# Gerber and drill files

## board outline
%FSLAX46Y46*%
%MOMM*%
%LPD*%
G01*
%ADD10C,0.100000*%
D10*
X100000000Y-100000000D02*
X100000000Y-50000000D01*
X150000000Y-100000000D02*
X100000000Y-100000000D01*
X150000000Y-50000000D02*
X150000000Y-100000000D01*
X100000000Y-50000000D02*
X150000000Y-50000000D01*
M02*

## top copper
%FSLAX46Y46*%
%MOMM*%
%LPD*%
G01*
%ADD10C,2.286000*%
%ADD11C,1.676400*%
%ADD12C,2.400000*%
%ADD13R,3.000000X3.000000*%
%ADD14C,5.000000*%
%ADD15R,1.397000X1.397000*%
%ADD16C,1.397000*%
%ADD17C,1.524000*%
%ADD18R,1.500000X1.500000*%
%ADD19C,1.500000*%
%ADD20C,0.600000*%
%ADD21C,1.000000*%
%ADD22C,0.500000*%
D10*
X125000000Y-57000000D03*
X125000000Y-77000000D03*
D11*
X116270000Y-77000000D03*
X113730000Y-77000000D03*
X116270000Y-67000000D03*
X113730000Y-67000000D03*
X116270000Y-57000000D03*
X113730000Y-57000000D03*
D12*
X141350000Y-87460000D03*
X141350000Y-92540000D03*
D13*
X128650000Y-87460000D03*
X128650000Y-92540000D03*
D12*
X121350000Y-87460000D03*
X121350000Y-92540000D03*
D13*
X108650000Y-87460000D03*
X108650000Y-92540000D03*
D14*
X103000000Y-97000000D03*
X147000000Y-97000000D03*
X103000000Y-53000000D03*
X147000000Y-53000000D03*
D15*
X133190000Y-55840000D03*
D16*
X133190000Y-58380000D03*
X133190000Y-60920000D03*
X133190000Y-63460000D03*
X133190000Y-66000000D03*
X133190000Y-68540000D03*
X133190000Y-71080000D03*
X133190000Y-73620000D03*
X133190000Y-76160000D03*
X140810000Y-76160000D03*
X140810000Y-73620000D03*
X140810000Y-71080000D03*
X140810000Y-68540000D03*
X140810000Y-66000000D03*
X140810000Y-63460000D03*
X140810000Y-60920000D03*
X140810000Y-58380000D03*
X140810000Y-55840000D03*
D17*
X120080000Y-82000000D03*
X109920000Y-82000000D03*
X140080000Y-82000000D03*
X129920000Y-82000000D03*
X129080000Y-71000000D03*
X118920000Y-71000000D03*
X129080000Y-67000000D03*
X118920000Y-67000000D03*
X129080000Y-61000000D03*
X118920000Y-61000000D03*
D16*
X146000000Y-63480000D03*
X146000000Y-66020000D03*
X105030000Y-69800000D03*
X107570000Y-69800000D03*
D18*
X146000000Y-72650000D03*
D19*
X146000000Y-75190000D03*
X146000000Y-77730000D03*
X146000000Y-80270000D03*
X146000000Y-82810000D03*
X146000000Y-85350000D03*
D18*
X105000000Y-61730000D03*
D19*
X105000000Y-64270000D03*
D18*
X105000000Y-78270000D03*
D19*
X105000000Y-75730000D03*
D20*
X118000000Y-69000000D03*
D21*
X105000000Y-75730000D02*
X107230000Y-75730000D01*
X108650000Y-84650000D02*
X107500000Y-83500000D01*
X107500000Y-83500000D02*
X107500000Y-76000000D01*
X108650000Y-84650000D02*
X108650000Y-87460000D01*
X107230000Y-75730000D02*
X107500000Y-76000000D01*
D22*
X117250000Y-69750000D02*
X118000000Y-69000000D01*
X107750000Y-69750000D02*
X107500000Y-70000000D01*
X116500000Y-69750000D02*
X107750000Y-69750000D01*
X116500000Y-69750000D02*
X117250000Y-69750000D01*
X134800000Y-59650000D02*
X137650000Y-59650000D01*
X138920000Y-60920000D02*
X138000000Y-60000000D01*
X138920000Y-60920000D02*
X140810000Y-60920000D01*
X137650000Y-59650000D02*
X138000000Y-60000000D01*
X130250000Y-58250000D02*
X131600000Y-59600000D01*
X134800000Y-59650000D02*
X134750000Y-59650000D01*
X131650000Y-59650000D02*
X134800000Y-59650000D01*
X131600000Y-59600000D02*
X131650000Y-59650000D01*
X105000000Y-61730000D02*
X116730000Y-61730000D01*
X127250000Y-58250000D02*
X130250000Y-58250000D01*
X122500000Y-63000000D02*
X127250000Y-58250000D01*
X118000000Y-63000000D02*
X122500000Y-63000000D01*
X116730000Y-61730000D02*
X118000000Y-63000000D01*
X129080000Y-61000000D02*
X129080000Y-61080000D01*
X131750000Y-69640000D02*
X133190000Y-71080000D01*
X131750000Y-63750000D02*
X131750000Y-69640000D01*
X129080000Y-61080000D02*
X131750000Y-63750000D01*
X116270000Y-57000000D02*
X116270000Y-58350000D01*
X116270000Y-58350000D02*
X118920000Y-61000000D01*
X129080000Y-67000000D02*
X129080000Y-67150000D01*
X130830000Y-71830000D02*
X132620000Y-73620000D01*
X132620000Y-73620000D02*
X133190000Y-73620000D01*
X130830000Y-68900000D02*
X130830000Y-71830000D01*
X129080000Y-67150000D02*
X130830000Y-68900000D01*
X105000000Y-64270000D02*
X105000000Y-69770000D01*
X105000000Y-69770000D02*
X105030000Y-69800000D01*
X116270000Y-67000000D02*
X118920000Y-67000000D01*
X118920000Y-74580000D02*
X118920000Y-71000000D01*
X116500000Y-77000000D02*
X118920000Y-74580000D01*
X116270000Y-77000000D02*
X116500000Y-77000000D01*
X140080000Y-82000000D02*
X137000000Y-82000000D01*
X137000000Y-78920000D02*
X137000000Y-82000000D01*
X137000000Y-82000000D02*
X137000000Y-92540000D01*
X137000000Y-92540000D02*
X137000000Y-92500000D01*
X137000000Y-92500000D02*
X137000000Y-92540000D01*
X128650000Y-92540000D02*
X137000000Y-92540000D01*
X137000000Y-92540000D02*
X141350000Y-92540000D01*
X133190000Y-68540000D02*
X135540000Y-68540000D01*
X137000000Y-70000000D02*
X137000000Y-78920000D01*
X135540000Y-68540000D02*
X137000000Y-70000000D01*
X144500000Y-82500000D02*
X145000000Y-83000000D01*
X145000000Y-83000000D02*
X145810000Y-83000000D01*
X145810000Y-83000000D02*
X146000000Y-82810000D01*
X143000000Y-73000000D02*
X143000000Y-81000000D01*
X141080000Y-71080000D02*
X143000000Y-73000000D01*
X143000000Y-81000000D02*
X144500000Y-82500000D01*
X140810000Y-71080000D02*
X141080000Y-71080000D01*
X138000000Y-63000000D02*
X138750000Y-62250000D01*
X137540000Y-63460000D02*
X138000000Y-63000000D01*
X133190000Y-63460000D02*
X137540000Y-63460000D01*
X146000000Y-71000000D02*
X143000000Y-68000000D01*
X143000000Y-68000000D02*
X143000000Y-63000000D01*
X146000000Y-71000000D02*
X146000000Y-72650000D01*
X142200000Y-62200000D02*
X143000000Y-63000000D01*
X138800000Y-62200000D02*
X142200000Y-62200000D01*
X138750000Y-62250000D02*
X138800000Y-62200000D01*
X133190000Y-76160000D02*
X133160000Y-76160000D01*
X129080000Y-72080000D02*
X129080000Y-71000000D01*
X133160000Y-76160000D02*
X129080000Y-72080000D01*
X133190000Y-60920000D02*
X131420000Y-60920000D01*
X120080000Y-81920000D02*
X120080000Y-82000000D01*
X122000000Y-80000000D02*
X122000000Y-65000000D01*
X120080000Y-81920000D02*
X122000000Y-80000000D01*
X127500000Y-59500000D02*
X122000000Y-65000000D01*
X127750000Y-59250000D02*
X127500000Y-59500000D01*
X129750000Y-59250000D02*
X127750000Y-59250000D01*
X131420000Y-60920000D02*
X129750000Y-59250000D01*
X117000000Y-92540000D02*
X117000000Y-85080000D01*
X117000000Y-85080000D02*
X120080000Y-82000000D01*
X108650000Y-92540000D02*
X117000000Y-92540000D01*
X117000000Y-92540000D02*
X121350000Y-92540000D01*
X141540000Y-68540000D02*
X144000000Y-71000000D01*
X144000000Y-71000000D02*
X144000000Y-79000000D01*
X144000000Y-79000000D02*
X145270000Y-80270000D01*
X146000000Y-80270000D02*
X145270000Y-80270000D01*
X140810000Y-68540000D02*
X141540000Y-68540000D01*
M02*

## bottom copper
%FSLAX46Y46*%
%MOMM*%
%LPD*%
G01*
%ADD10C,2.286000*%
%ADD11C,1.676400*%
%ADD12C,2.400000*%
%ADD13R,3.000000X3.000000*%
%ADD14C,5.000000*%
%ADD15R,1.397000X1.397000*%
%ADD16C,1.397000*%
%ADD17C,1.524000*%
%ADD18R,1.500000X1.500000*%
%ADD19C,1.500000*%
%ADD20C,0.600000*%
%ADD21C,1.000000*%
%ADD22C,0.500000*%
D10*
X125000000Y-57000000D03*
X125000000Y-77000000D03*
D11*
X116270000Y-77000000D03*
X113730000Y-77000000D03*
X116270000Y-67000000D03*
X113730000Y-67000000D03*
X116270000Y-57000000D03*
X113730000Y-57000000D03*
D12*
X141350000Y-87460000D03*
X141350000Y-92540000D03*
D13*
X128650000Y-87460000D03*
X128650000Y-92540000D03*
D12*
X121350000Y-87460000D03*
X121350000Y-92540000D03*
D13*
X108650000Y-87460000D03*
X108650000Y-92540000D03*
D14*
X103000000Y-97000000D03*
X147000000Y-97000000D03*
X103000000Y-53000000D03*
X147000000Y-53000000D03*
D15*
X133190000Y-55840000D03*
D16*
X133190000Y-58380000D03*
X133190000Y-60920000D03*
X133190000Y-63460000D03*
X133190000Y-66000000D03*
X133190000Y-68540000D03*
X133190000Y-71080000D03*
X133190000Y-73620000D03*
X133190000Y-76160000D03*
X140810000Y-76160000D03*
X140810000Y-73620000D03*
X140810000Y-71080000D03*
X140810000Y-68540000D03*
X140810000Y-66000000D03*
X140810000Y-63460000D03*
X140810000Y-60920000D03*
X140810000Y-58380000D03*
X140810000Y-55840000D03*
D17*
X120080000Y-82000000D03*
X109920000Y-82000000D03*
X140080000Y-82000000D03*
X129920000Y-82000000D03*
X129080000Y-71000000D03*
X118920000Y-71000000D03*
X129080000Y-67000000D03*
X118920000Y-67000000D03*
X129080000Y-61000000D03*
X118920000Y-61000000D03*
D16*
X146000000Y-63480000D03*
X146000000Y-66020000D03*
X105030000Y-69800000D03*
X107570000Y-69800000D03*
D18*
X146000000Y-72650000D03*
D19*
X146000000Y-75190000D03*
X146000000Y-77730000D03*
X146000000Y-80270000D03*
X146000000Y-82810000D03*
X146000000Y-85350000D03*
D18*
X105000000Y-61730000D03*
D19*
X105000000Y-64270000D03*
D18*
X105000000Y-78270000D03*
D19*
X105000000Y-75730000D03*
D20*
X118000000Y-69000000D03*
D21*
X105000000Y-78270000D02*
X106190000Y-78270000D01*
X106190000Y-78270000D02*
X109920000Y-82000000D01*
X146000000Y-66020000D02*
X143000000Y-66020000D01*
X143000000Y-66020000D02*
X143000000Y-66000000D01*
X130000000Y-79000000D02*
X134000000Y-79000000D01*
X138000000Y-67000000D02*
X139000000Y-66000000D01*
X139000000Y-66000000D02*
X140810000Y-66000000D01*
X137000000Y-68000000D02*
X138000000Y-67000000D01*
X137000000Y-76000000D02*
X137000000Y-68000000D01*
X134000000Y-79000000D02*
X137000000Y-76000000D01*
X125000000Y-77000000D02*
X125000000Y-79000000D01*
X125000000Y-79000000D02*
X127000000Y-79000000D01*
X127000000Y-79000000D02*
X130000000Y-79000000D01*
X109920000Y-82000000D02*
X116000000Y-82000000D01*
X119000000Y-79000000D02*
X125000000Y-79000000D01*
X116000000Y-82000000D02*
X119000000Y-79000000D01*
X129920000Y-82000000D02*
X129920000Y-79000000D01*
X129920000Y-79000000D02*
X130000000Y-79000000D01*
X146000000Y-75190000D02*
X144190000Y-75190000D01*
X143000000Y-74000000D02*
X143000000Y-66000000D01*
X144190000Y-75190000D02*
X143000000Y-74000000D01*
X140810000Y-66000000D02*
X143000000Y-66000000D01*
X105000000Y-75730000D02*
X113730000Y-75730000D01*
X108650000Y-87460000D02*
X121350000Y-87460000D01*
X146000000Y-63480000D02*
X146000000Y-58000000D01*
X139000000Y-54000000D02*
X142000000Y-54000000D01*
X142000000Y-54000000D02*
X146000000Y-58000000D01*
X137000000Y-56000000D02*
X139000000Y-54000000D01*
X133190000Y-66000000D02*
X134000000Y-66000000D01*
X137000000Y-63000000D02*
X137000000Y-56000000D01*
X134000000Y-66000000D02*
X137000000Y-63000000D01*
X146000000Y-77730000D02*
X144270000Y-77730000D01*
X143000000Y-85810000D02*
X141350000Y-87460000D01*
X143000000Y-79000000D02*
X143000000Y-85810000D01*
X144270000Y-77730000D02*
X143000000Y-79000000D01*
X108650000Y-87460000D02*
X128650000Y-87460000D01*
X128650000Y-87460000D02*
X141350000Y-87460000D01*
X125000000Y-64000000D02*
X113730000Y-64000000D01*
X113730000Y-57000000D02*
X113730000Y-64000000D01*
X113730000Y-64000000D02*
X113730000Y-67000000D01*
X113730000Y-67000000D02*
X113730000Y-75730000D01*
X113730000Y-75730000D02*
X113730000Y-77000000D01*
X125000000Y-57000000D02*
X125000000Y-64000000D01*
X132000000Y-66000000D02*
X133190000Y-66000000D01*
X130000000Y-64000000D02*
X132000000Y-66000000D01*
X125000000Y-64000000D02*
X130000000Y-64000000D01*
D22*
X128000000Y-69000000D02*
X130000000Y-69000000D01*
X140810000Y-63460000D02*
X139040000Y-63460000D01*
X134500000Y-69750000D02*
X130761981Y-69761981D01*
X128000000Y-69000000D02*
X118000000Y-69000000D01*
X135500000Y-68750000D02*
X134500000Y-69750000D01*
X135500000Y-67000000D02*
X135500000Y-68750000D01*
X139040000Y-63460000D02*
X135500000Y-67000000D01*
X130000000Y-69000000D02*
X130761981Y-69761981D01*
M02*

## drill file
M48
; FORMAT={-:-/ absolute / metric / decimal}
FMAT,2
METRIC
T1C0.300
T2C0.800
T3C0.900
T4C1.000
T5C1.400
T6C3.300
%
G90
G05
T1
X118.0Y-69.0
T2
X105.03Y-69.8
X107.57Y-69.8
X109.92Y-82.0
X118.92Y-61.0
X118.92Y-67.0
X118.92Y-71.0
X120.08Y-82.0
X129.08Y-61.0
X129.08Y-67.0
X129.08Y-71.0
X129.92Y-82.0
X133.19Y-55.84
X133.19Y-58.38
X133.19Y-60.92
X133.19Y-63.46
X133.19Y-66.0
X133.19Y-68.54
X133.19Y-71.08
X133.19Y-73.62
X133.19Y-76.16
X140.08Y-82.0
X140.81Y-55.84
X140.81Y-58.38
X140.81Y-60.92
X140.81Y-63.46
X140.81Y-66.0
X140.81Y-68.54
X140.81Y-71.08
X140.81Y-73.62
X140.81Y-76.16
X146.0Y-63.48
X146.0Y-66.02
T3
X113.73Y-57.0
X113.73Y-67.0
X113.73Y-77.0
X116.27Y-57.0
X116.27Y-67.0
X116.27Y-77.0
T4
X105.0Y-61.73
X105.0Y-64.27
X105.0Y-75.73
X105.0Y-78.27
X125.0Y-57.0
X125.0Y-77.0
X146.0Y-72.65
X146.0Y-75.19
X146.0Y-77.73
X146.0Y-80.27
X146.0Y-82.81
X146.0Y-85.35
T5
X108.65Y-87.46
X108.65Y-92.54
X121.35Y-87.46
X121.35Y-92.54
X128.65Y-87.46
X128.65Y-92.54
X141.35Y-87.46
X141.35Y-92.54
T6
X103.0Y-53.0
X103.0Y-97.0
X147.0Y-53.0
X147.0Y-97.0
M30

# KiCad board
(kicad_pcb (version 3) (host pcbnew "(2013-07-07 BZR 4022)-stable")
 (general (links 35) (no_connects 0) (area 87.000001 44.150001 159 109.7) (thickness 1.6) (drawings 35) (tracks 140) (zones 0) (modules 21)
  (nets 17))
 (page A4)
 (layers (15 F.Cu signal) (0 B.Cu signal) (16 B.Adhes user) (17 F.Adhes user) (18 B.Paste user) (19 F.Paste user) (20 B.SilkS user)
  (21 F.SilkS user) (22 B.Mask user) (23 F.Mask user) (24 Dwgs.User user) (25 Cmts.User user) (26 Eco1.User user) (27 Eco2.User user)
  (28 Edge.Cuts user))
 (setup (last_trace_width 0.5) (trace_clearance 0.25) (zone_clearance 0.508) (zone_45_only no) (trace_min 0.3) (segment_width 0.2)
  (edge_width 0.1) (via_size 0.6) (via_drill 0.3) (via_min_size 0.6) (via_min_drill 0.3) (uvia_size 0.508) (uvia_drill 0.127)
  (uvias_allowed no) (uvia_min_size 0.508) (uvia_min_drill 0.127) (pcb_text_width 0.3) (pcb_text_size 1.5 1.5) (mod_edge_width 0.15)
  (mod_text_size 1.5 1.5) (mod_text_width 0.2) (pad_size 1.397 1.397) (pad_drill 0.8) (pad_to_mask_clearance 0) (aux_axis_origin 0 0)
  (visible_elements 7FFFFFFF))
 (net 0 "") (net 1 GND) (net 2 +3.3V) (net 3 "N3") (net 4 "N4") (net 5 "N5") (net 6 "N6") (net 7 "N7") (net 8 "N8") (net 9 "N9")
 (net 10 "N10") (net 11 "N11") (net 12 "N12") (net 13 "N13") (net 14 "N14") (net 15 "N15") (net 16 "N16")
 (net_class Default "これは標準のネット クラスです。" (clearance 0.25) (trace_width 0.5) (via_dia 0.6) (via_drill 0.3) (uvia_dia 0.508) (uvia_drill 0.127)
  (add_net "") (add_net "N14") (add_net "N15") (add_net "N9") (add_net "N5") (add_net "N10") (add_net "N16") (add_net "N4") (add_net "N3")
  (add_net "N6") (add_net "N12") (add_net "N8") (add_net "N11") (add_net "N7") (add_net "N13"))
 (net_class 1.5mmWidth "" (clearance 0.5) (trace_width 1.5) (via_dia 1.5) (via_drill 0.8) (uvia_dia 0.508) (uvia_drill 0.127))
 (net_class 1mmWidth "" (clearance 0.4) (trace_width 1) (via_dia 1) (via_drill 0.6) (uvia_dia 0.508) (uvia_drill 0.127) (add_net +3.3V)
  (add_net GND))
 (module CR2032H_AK (layer B.Cu) (at 125 62 270)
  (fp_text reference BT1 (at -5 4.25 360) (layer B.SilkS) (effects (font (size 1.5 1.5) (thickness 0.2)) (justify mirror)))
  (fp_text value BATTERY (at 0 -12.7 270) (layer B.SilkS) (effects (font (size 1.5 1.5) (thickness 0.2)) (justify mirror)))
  (pad 2 thru_hole circle (at -5 0 270) (size 2.286 2.286) (drill 1) (layers *.Cu *.Mask B.SilkS) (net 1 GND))
  (pad 1 thru_hole circle (at 15 0 270) (size 2.286 2.286) (drill 1) (layers *.Cu *.Mask B.SilkS) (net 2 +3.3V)))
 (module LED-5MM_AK (layer F.Cu) (at 115 77 180)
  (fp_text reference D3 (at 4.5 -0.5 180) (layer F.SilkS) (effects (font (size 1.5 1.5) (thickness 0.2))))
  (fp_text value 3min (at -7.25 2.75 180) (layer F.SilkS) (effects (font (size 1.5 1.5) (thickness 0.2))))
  (pad 1 thru_hole circle (at -1.27 0 180) (size 1.6764 1.6764) (drill 0.9) (layers *.Cu *.Mask F.SilkS) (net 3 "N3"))
  (pad 2 thru_hole circle (at 1.27 0 180) (size 1.6764 1.6764) (drill 0.9) (layers *.Cu *.Mask F.SilkS) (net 1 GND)))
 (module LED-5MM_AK (layer F.Cu) (at 115 67 180)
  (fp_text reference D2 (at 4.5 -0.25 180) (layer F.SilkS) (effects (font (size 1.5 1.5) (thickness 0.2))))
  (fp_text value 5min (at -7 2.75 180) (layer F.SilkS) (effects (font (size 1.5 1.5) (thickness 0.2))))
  (pad 1 thru_hole circle (at -1.27 0 180) (size 1.6764 1.6764) (drill 0.9) (layers *.Cu *.Mask F.SilkS) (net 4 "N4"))
  (pad 2 thru_hole circle (at 1.27 0 180) (size 1.6764 1.6764) (drill 0.9) (layers *.Cu *.Mask F.SilkS) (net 1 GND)))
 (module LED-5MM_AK (layer F.Cu) (at 115 57 180)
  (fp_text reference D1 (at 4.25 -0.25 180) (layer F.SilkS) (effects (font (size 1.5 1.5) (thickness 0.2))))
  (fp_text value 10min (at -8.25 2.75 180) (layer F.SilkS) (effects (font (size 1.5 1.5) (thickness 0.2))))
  (pad 1 thru_hole circle (at -1.27 0 180) (size 1.6764 1.6764) (drill 0.9) (layers *.Cu *.Mask F.SilkS) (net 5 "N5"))
  (pad 2 thru_hole circle (at 1.27 0 180) (size 1.6764 1.6764) (drill 0.9) (layers *.Cu *.Mask F.SilkS) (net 1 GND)))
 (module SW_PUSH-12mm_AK (layer F.Cu) (at 135 90)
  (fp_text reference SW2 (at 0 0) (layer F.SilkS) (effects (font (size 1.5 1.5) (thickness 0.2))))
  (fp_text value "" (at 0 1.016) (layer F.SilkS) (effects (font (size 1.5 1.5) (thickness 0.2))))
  (pad 1 thru_hole circle (at 6.35 -2.54) (size 2.4 2.4) (drill 1.4) (layers *.Cu *.Mask F.SilkS) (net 1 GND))
  (pad 2 thru_hole circle (at 6.35 2.54) (size 2.4 2.4) (drill 1.4) (layers *.Cu *.Mask F.SilkS) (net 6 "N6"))
  (pad 1 thru_hole rect (at -6.35 -2.54) (size 3 3) (drill 1.4) (layers *.Cu *.Mask F.SilkS) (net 1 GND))
  (pad 2 thru_hole rect (at -6.35 2.54) (size 3 3) (drill 1.4) (layers *.Cu *.Mask F.SilkS) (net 6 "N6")))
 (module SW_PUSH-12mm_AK (layer F.Cu) (at 115 90)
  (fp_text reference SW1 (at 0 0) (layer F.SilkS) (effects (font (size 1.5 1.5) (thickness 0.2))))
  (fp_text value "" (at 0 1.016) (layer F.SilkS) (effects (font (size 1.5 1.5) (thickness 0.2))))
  (pad 1 thru_hole circle (at 6.35 -2.54) (size 2.4 2.4) (drill 1.4) (layers *.Cu *.Mask F.SilkS) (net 1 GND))
  (pad 2 thru_hole circle (at 6.35 2.54) (size 2.4 2.4) (drill 1.4) (layers *.Cu *.Mask F.SilkS) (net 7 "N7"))
  (pad 1 thru_hole rect (at -6.35 -2.54) (size 3 3) (drill 1.4) (layers *.Cu *.Mask F.SilkS) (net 1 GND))
  (pad 2 thru_hole rect (at -6.35 2.54) (size 3 3) (drill 1.4) (layers *.Cu *.Mask F.SilkS) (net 7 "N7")))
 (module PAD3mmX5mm (layer F.Cu) (at 103 97)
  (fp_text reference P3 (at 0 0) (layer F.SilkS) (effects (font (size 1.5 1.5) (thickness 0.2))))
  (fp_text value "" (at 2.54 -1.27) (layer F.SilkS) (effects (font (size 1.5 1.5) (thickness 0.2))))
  (pad "" thru_hole circle (at 0 0) (size 5 5) (drill 3.3) (layers *.Cu *.Mask F.SilkS)))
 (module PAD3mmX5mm (layer F.Cu) (at 147 97)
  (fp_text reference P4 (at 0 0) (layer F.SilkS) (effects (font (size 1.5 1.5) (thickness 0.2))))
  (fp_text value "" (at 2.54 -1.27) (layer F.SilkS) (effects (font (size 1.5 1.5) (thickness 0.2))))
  (pad "" thru_hole circle (at 0 0) (size 5 5) (drill 3.3) (layers *.Cu *.Mask F.SilkS)))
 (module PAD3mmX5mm (layer F.Cu) (at 103 53)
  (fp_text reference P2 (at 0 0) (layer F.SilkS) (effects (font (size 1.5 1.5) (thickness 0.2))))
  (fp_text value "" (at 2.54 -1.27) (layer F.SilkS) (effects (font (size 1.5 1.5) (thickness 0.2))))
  (pad "" thru_hole circle (at 0 0) (size 5 5) (drill 3.3) (layers *.Cu *.Mask F.SilkS)))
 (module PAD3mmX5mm (layer F.Cu) (at 147 53)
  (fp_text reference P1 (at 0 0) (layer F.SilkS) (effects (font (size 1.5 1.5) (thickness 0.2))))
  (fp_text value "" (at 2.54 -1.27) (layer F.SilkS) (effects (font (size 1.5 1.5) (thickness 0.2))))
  (pad "" thru_hole circle (at 0 0) (size 5 5) (drill 3.3) (layers *.Cu *.Mask F.SilkS)))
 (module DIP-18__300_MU (layer F.Cu) (at 137 66 270)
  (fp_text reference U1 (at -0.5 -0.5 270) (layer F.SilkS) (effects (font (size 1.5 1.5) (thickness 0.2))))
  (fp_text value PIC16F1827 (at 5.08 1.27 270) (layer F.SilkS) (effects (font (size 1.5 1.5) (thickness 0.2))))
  (pad 1 thru_hole rect (at -10.16 3.81 270) (size 1.397 1.397) (drill 0.8) (layers *.Cu *.Mask F.SilkS))
  (pad 2 thru_hole circle (at -7.62 3.81 270) (size 1.397 1.397) (drill 0.8) (layers *.Cu *.Mask F.SilkS))
  (pad 3 thru_hole circle (at -5.08 3.81 270) (size 1.397 1.397) (drill 0.8) (layers *.Cu *.Mask F.SilkS) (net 7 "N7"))
  (pad 4 thru_hole circle (at -2.54 3.81 270) (size 1.397 1.397) (drill 0.8) (layers *.Cu *.Mask F.SilkS) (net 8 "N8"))
  (pad 5 thru_hole circle (at 0 3.81 270) (size 1.397 1.397) (drill 0.8) (layers *.Cu *.Mask F.SilkS) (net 1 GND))
  (pad 6 thru_hole circle (at 2.54 3.81 270) (size 1.397 1.397) (drill 0.8) (layers *.Cu *.Mask F.SilkS) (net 6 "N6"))
  (pad 7 thru_hole circle (at 5.08 3.81 270) (size 1.397 1.397) (drill 0.8) (layers *.Cu *.Mask F.SilkS) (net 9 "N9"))
  (pad 8 thru_hole circle (at 7.62 3.81 270) (size 1.397 1.397) (drill 0.8) (layers *.Cu *.Mask F.SilkS) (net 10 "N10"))
  (pad 9 thru_hole circle (at 10.16 3.81 270) (size 1.397 1.397) (drill 0.8) (layers *.Cu *.Mask F.SilkS) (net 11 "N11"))
  (pad 10 thru_hole circle (at 10.16 -3.81 270) (size 1.397 1.397) (drill 0.8) (layers *.Cu *.Mask F.SilkS))
  (pad 11 thru_hole circle (at 7.62 -3.81 270) (size 1.397 1.397) (drill 0.8) (layers *.Cu *.Mask F.SilkS))
  (pad 12 thru_hole circle (at 5.08 -3.81 270) (size 1.397 1.397) (drill 0.8) (layers *.Cu *.Mask F.SilkS) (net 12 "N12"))
  (pad 13 thru_hole circle (at 2.54 -3.81 270) (size 1.397 1.397) (drill 0.8) (layers *.Cu *.Mask F.SilkS) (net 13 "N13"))
  (pad 14 thru_hole circle (at 0 -3.81 270) (size 1.397 1.397) (drill 0.8) (layers *.Cu *.Mask F.SilkS) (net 2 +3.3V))
  (pad 15 thru_hole circle (at -2.54 -3.81 270) (size 1.397 1.397) (drill 0.8) (layers *.Cu *.Mask F.SilkS) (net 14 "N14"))
  (pad 16 thru_hole circle (at -5.08 -3.81 270) (size 1.397 1.397) (drill 0.8) (layers *.Cu *.Mask F.SilkS) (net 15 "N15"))
  (pad 17 thru_hole circle (at -7.62 -3.81 270) (size 1.397 1.397) (drill 0.8) (layers *.Cu *.Mask F.SilkS))
  (pad 18 thru_hole circle (at -10.16 -3.81 270) (size 1.397 1.397) (drill 0.8) (layers *.Cu *.Mask F.SilkS)))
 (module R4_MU (layer F.Cu) (at 115 82 180) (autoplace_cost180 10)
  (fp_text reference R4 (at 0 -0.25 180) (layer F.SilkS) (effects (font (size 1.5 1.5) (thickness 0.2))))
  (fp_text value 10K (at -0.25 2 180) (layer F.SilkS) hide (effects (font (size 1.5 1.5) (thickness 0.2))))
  (pad 1 thru_hole circle (at -5.08 0 180) (size 1.524 1.524) (drill 0.8) (layers *.Cu *.Mask F.SilkS) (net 7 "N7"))
  (pad 2 thru_hole circle (at 5.08 0 180) (size 1.524 1.524) (drill 0.8) (layers *.Cu *.Mask F.SilkS) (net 2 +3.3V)))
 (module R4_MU (layer F.Cu) (at 135 82 180) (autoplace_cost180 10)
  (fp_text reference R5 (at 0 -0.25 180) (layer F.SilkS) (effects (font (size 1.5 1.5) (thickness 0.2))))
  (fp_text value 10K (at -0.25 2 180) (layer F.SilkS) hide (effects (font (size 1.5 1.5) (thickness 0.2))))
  (pad 1 thru_hole circle (at -5.08 0 180) (size 1.524 1.524) (drill 0.8) (layers *.Cu *.Mask F.SilkS) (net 6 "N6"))
  (pad 2 thru_hole circle (at 5.08 0 180) (size 1.524 1.524) (drill 0.8) (layers *.Cu *.Mask F.SilkS) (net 2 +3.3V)))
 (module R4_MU (layer F.Cu) (at 124 71 180) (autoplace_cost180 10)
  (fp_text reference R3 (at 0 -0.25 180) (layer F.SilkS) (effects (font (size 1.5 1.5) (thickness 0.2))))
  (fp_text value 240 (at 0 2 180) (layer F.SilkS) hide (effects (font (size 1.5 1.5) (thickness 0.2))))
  (pad 1 thru_hole circle (at -5.08 0 180) (size 1.524 1.524) (drill 0.8) (layers *.Cu *.Mask F.SilkS) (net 11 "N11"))
  (pad 2 thru_hole circle (at 5.08 0 180) (size 1.524 1.524) (drill 0.8) (layers *.Cu *.Mask F.SilkS) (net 3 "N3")))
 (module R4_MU (layer F.Cu) (at 124 67 180) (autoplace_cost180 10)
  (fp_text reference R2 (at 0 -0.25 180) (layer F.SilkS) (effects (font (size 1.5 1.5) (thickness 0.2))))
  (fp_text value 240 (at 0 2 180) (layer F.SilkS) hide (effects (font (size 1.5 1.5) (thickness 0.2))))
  (pad 1 thru_hole circle (at -5.08 0 180) (size 1.524 1.524) (drill 0.8) (layers *.Cu *.Mask F.SilkS) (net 10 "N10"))
  (pad 2 thru_hole circle (at 5.08 0 180) (size 1.524 1.524) (drill 0.8) (layers *.Cu *.Mask F.SilkS) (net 4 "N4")))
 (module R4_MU (layer F.Cu) (at 124 61 180) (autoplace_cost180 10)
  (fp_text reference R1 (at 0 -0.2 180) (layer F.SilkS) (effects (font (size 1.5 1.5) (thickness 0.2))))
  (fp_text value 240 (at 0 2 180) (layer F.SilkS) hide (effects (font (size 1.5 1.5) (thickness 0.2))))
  (pad 1 thru_hole circle (at -5.08 0 180) (size 1.524 1.524) (drill 0.8) (layers *.Cu *.Mask F.SilkS) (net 9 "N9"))
  (pad 2 thru_hole circle (at 5.08 0 180) (size 1.524 1.524) (drill 0.8) (layers *.Cu *.Mask F.SilkS) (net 5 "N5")))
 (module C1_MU (layer F.Cu) (at 146 64.75 270)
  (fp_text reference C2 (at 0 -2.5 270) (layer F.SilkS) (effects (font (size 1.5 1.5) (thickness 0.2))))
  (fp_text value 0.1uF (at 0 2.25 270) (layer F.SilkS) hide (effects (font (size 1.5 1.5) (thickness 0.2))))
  (pad 1 thru_hole circle (at -1.27 0 270) (size 1.397 1.397) (drill 0.8) (layers *.Cu *.Mask F.SilkS) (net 1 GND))
  (pad 2 thru_hole circle (at 1.27 0 270) (size 1.397 1.397) (drill 0.8) (layers *.Cu *.Mask F.SilkS) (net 2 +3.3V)))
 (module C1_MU (layer F.Cu) (at 106.3 69.8)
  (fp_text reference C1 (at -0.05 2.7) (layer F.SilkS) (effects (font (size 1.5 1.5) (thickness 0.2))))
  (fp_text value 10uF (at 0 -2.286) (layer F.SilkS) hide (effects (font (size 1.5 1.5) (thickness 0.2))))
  (pad 1 thru_hole circle (at -1.27 0) (size 1.397 1.397) (drill 0.8) (layers *.Cu *.Mask F.SilkS) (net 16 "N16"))
  (pad 2 thru_hole circle (at 1.27 0) (size 1.397 1.397) (drill 0.8) (layers *.Cu *.Mask F.SilkS) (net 14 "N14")))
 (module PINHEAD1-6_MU (layer F.Cu) (at 146 79 270)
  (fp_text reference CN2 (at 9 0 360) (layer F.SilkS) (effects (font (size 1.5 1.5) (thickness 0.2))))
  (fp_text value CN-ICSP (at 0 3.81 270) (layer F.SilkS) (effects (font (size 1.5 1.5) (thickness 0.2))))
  (pad 1 thru_hole rect (at -6.35 0 270) (size 1.5 1.5) (drill 1) (layers *.Cu *.Mask F.SilkS) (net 8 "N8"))
  (pad 2 thru_hole circle (at -3.81 0 270) (size 1.5 1.5) (drill 1) (layers *.Cu *.Mask F.SilkS) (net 2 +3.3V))
  (pad 3 thru_hole circle (at -1.27 0 270) (size 1.5 1.5) (drill 1) (layers *.Cu *.Mask F.SilkS) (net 1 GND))
  (pad 4 thru_hole circle (at 1.27 0 270) (size 1.5 1.5) (drill 1) (layers *.Cu *.Mask F.SilkS) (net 13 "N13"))
  (pad 5 thru_hole circle (at 3.81 0 270) (size 1.5 1.5) (drill 1) (layers *.Cu *.Mask F.SilkS) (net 12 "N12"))
  (pad 6 thru_hole circle (at 6.35 0 270) (size 1.5 1.5) (drill 1) (layers *.Cu *.Mask F.SilkS)))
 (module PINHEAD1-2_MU (layer F.Cu) (at 105 63 270)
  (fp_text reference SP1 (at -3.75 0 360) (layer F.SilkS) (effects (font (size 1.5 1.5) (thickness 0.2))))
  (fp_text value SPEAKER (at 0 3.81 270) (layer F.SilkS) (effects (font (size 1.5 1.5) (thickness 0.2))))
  (pad 1 thru_hole rect (at -1.27 0 270) (size 1.5 1.5) (drill 1) (layers *.Cu *.Mask F.SilkS) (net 15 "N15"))
  (pad 2 thru_hole circle (at 1.27 0 270) (size 1.5 1.5) (drill 1) (layers *.Cu *.Mask F.SilkS) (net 16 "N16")))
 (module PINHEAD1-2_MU (layer B.Cu) (at 105 77 90)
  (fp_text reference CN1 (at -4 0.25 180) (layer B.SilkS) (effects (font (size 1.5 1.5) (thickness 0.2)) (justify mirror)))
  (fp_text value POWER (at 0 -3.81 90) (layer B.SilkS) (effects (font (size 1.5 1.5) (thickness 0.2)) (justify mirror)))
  (pad 1 thru_hole rect (at -1.27 0 90) (size 1.5 1.5) (drill 1) (layers *.Cu *.Mask B.SilkS) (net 2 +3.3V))
  (pad 2 thru_hole circle (at 1.27 0 90) (size 1.5 1.5) (drill 1) (layers *.Cu *.Mask B.SilkS) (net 1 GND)))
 (gr_line (start 100 100) (end 100 50) (angle 90) (layer Edge.Cuts) (width 0.1))
 (gr_line (start 150 100) (end 100 100) (angle 90) (layer Edge.Cuts) (width 0.1))
 (gr_line (start 150 50) (end 150 100) (angle 90) (layer Edge.Cuts) (width 0.1))
 (gr_line (start 100 50) (end 150 50) (angle 90) (layer Edge.Cuts) (width 0.1))
 (segment (start 105 78.27) (end 106.19 78.27) (width 1) (layer B.Cu) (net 2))
 (segment (start 106.19 78.27) (end 109.92 82) (width 1) (layer B.Cu) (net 2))
 (segment (start 146 66.02) (end 143 66.02) (width 1) (layer B.Cu) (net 2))
 (segment (start 143 66.02) (end 143 66) (width 1) (layer B.Cu) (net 2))
 (segment (start 130 79) (end 134 79) (width 1) (layer B.Cu) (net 2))
 (segment (start 138 67) (end 139 66) (width 1) (layer B.Cu) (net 2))
 (segment (start 139 66) (end 140.81 66) (width 1) (layer B.Cu) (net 2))
 (segment (start 137 68) (end 138 67) (width 1) (layer B.Cu) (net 2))
 (segment (start 137 76) (end 137 68) (width 1) (layer B.Cu) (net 2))
 (segment (start 134 79) (end 137 76) (width 1) (layer B.Cu) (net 2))
 (segment (start 125 77) (end 125 79) (width 1) (layer B.Cu) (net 2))
 (segment (start 125 79) (end 127 79) (width 1) (layer B.Cu) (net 2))
 (segment (start 127 79) (end 130 79) (width 1) (layer B.Cu) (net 2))
 (segment (start 109.92 82) (end 116 82) (width 1) (layer B.Cu) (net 2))
 (segment (start 119 79) (end 125 79) (width 1) (layer B.Cu) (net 2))
 (segment (start 116 82) (end 119 79) (width 1) (layer B.Cu) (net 2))
 (segment (start 129.92 82) (end 129.92 79) (width 1) (layer B.Cu) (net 2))
 (segment (start 129.92 79) (end 130 79) (width 1) (layer B.Cu) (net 2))
 (segment (start 146 75.19) (end 144.19 75.19) (width 1) (layer B.Cu) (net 2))
 (segment (start 143 74) (end 143 66) (width 1) (layer B.Cu) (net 2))
 (segment (start 144.19 75.19) (end 143 74) (width 1) (layer B.Cu) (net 2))
 (segment (start 140.81 66) (end 143 66) (width 1) (layer B.Cu) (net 2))
 (segment (start 105 75.73) (end 107.23 75.73) (width 1) (layer F.Cu) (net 1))
 (segment (start 108.65 84.65) (end 107.5 83.5) (width 1) (layer F.Cu) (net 1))
 (segment (start 107.5 83.5) (end 107.5 76) (width 1) (layer F.Cu) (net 1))
 (segment (start 108.65 84.65) (end 108.65 87.46) (width 1) (layer F.Cu) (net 1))
 (segment (start 107.23 75.73) (end 107.5 76) (width 1) (layer F.Cu) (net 1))
 (segment (start 105 75.73) (end 113.73 75.73) (width 1) (layer B.Cu) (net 1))
 (segment (start 108.65 87.46) (end 121.35 87.46) (width 1) (layer B.Cu) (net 1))
 (segment (start 146 63.48) (end 146 58) (width 1) (layer B.Cu) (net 1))
 (segment (start 139 54) (end 142 54) (width 1) (layer B.Cu) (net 1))
 (segment (start 142 54) (end 146 58) (width 1) (layer B.Cu) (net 1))
 (segment (start 137 56) (end 139 54) (width 1) (layer B.Cu) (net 1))
 (segment (start 133.19 66) (end 134 66) (width 1) (layer B.Cu) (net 1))
 (segment (start 137 63) (end 137 56) (width 1) (layer B.Cu) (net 1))
 (segment (start 134 66) (end 137 63) (width 1) (layer B.Cu) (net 1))
 (segment (start 146 77.73) (end 144.27 77.73) (width 1) (layer B.Cu) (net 1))
 (segment (start 143 85.81) (end 141.35 87.46) (width 1) (layer B.Cu) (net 1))
 (segment (start 143 79) (end 143 85.81) (width 1) (layer B.Cu) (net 1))
 (segment (start 144.27 77.73) (end 143 79) (width 1) (layer B.Cu) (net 1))
 (segment (start 108.65 87.46) (end 128.65 87.46) (width 1) (layer B.Cu) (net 1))
 (segment (start 128.65 87.46) (end 141.35 87.46) (width 1) (layer B.Cu) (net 1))
 (segment (start 125 64) (end 113.73 64) (width 1) (layer B.Cu) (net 1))
 (segment (start 113.73 57) (end 113.73 64) (width 1) (layer B.Cu) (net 1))
 (segment (start 113.73 64) (end 113.73 67) (width 1) (layer B.Cu) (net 1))
 (segment (start 113.73 67) (end 113.73 75.73) (width 1) (layer B.Cu) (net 1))
 (segment (start 113.73 75.73) (end 113.73 77) (width 1) (layer B.Cu) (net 1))
 (segment (start 125 57) (end 125 64) (width 1) (layer B.Cu) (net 1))
 (segment (start 132 66) (end 133.19 66) (width 1) (layer B.Cu) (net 1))
 (segment (start 130 64) (end 132 66) (width 1) (layer B.Cu) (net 1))
 (segment (start 125 64) (end 130 64) (width 1) (layer B.Cu) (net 1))
 (segment (start 128 69) (end 130 69) (width 0.5) (layer B.Cu) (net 14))
 (segment (start 117.25 69.75) (end 118 69) (width 0.5) (layer F.Cu) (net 14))
 (segment (start 140.81 63.46) (end 139.04 63.46) (width 0.5) (layer B.Cu) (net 14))
 (segment (start 107.75 69.75) (end 107.5 70) (width 0.5) (layer F.Cu) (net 14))
 (segment (start 116.5 69.75) (end 107.75 69.75) (width 0.5) (layer F.Cu) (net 14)) (via (at 118 69) (size 0.6) (layers F.Cu B.Cu) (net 14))
 (segment (start 134.5 69.75) (end 130.761981 69.761981) (width 0.5) (layer B.Cu) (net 14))
 (segment (start 128 69) (end 118 69) (width 0.5) (layer B.Cu) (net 14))
 (segment (start 135.5 68.75) (end 134.5 69.75) (width 0.5) (layer B.Cu) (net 14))
 (segment (start 135.5 67) (end 135.5 68.75) (width 0.5) (layer B.Cu) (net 14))
 (segment (start 139.04 63.46) (end 135.5 67) (width 0.5) (layer B.Cu) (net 14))
 (segment (start 116.5 69.75) (end 117.25 69.75) (width 0.5) (layer F.Cu) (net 14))
 (segment (start 130 69) (end 130.761981 69.761981) (width 0.5) (layer B.Cu) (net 14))
 (segment (start 134.8 59.65) (end 137.65 59.65) (width 0.5) (layer F.Cu) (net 15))
 (segment (start 138.92 60.92) (end 138 60) (width 0.5) (layer F.Cu) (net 15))
 (segment (start 138.92 60.92) (end 140.81 60.92) (width 0.5) (layer F.Cu) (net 15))
 (segment (start 137.65 59.65) (end 138 60) (width 0.5) (layer F.Cu) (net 15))
 (segment (start 130.25 58.25) (end 131.6 59.6) (width 0.5) (layer F.Cu) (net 15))
 (segment (start 134.8 59.65) (end 134.75 59.65) (width 0.5) (layer F.Cu) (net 15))
 (segment (start 131.65 59.65) (end 134.8 59.65) (width 0.5) (layer F.Cu) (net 15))
 (segment (start 131.6 59.6) (end 131.65 59.65) (width 0.5) (layer F.Cu) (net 15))
 (segment (start 105 61.73) (end 116.73 61.73) (width 0.5) (layer F.Cu) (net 15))
 (segment (start 127.25 58.25) (end 130.25 58.25) (width 0.5) (layer F.Cu) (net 15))
 (segment (start 122.5 63) (end 127.25 58.25) (width 0.5) (layer F.Cu) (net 15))
 (segment (start 118 63) (end 122.5 63) (width 0.5) (layer F.Cu) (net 15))
 (segment (start 116.73 61.73) (end 118 63) (width 0.5) (layer F.Cu) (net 15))
 (segment (start 129.08 61) (end 129.08 61.08) (width 0.5) (layer F.Cu) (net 9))
 (segment (start 131.75 69.64) (end 133.19 71.08) (width 0.5) (layer F.Cu) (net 9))
 (segment (start 131.75 63.75) (end 131.75 69.64) (width 0.5) (layer F.Cu) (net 9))
 (segment (start 129.08 61.08) (end 131.75 63.75) (width 0.5) (layer F.Cu) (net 9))
 (segment (start 116.27 57) (end 116.27 58.35) (width 0.5) (layer F.Cu) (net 5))
 (segment (start 116.27 58.35) (end 118.92 61) (width 0.5) (layer F.Cu) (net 5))
 (segment (start 129.08 67) (end 129.08 67.15) (width 0.5) (layer F.Cu) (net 10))
 (segment (start 130.83 71.83) (end 132.62 73.62) (width 0.5) (layer F.Cu) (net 10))
 (segment (start 132.62 73.62) (end 133.19 73.62) (width 0.5) (layer F.Cu) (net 10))
 (segment (start 130.83 68.9) (end 130.83 71.83) (width 0.5) (layer F.Cu) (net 10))
 (segment (start 129.08 67.15) (end 130.83 68.9) (width 0.5) (layer F.Cu) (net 10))
 (segment (start 105 64.27) (end 105 69.77) (width 0.5) (layer F.Cu) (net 16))
 (segment (start 105 69.77) (end 105.03 69.8) (width 0.5) (layer F.Cu) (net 16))
 (segment (start 116.27 67) (end 118.92 67) (width 0.5) (layer F.Cu) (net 4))
 (segment (start 118.92 74.58) (end 118.92 71) (width 0.5) (layer F.Cu) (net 3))
 (segment (start 116.5 77) (end 118.92 74.58) (width 0.5) (layer F.Cu) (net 3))
 (segment (start 116.27 77) (end 116.5 77) (width 0.5) (layer F.Cu) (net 3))
 (segment (start 140.08 82) (end 137 82) (width 0.5) (layer F.Cu) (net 6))
 (segment (start 137 78.92) (end 137 82) (width 0.5) (layer F.Cu) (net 6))
 (segment (start 137 82) (end 137 92.54) (width 0.5) (layer F.Cu) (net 6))
 (segment (start 137 92.54) (end 137 92.5) (width 0.5) (layer F.Cu) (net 6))
 (segment (start 137 92.5) (end 137 92.54) (width 0.5) (layer F.Cu) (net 6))
 (segment (start 128.65 92.54) (end 137 92.54) (width 0.5) (layer F.Cu) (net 6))
 (segment (start 137 92.54) (end 141.35 92.54) (width 0.5) (layer F.Cu) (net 6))
 (segment (start 133.19 68.54) (end 135.54 68.54) (width 0.5) (layer F.Cu) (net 6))
 (segment (start 137 70) (end 137 78.92) (width 0.5) (layer F.Cu) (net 6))
 (segment (start 135.54 68.54) (end 137 70) (width 0.5) (layer F.Cu) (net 6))
 (segment (start 144.5 82.5) (end 145 83) (width 0.5) (layer F.Cu) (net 12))
 (segment (start 145 83) (end 145.81 83) (width 0.5) (layer F.Cu) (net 12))
 (segment (start 145.81 83) (end 146 82.81) (width 0.5) (layer F.Cu) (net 12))
 (segment (start 143 73) (end 143 81) (width 0.5) (layer F.Cu) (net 12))
 (segment (start 141.08 71.08) (end 143 73) (width 0.5) (layer F.Cu) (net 12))
 (segment (start 143 81) (end 144.5 82.5) (width 0.5) (layer F.Cu) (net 12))
 (segment (start 140.81 71.08) (end 141.08 71.08) (width 0.5) (layer F.Cu) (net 12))
 (segment (start 138 63) (end 138.75 62.25) (width 0.5) (layer F.Cu) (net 8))
 (segment (start 137.54 63.46) (end 138 63) (width 0.5) (layer F.Cu) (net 8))
 (segment (start 133.19 63.46) (end 137.54 63.46) (width 0.5) (layer F.Cu) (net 8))
 (segment (start 146 71) (end 143 68) (width 0.5) (layer F.Cu) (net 8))
 (segment (start 143 68) (end 143 63) (width 0.5) (layer F.Cu) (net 8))
 (segment (start 146 71) (end 146 72.65) (width 0.5) (layer F.Cu) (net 8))
 (segment (start 142.2 62.2) (end 143 63) (width 0.5) (layer F.Cu) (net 8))
 (segment (start 138.8 62.2) (end 142.2 62.2) (width 0.5) (layer F.Cu) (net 8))
 (segment (start 138.75 62.25) (end 138.8 62.2) (width 0.5) (layer F.Cu) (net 8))
 (segment (start 133.19 76.16) (end 133.16 76.16) (width 0.5) (layer F.Cu) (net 11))
 (segment (start 129.08 72.08) (end 129.08 71) (width 0.5) (layer F.Cu) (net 11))
 (segment (start 133.16 76.16) (end 129.08 72.08) (width 0.5) (layer F.Cu) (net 11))
 (segment (start 133.19 60.92) (end 131.42 60.92) (width 0.5) (layer F.Cu) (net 7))
 (segment (start 120.08 81.92) (end 120.08 82) (width 0.5) (layer F.Cu) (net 7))
 (segment (start 122 80) (end 122 65) (width 0.5) (layer F.Cu) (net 7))
 (segment (start 120.08 81.92) (end 122 80) (width 0.5) (layer F.Cu) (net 7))
 (segment (start 127.5 59.5) (end 122 65) (width 0.5) (layer F.Cu) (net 7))
 (segment (start 127.75 59.25) (end 127.5 59.5) (width 0.5) (layer F.Cu) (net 7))
 (segment (start 129.75 59.25) (end 127.75 59.25) (width 0.5) (layer F.Cu) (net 7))
 (segment (start 131.42 60.92) (end 129.75 59.25) (width 0.5) (layer F.Cu) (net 7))
 (segment (start 117 92.54) (end 117 85.08) (width 0.5) (layer F.Cu) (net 7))
 (segment (start 117 85.08) (end 120.08 82) (width 0.5) (layer F.Cu) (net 7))
 (segment (start 108.65 92.54) (end 117 92.54) (width 0.5) (layer F.Cu) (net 7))
 (segment (start 117 92.54) (end 121.35 92.54) (width 0.5) (layer F.Cu) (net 7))
 (segment (start 141.54 68.54) (end 144 71) (width 0.5) (layer F.Cu) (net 13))
 (segment (start 144 71) (end 144 79) (width 0.5) (layer F.Cu) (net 13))
 (segment (start 144 79) (end 145.27 80.27) (width 0.5) (layer F.Cu) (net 13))
 (segment (start 146 80.27) (end 145.27 80.27) (width 0.5) (layer F.Cu) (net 13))
 (segment (start 140.81 68.54) (end 141.54 68.54) (width 0.5) (layer F.Cu) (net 13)))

